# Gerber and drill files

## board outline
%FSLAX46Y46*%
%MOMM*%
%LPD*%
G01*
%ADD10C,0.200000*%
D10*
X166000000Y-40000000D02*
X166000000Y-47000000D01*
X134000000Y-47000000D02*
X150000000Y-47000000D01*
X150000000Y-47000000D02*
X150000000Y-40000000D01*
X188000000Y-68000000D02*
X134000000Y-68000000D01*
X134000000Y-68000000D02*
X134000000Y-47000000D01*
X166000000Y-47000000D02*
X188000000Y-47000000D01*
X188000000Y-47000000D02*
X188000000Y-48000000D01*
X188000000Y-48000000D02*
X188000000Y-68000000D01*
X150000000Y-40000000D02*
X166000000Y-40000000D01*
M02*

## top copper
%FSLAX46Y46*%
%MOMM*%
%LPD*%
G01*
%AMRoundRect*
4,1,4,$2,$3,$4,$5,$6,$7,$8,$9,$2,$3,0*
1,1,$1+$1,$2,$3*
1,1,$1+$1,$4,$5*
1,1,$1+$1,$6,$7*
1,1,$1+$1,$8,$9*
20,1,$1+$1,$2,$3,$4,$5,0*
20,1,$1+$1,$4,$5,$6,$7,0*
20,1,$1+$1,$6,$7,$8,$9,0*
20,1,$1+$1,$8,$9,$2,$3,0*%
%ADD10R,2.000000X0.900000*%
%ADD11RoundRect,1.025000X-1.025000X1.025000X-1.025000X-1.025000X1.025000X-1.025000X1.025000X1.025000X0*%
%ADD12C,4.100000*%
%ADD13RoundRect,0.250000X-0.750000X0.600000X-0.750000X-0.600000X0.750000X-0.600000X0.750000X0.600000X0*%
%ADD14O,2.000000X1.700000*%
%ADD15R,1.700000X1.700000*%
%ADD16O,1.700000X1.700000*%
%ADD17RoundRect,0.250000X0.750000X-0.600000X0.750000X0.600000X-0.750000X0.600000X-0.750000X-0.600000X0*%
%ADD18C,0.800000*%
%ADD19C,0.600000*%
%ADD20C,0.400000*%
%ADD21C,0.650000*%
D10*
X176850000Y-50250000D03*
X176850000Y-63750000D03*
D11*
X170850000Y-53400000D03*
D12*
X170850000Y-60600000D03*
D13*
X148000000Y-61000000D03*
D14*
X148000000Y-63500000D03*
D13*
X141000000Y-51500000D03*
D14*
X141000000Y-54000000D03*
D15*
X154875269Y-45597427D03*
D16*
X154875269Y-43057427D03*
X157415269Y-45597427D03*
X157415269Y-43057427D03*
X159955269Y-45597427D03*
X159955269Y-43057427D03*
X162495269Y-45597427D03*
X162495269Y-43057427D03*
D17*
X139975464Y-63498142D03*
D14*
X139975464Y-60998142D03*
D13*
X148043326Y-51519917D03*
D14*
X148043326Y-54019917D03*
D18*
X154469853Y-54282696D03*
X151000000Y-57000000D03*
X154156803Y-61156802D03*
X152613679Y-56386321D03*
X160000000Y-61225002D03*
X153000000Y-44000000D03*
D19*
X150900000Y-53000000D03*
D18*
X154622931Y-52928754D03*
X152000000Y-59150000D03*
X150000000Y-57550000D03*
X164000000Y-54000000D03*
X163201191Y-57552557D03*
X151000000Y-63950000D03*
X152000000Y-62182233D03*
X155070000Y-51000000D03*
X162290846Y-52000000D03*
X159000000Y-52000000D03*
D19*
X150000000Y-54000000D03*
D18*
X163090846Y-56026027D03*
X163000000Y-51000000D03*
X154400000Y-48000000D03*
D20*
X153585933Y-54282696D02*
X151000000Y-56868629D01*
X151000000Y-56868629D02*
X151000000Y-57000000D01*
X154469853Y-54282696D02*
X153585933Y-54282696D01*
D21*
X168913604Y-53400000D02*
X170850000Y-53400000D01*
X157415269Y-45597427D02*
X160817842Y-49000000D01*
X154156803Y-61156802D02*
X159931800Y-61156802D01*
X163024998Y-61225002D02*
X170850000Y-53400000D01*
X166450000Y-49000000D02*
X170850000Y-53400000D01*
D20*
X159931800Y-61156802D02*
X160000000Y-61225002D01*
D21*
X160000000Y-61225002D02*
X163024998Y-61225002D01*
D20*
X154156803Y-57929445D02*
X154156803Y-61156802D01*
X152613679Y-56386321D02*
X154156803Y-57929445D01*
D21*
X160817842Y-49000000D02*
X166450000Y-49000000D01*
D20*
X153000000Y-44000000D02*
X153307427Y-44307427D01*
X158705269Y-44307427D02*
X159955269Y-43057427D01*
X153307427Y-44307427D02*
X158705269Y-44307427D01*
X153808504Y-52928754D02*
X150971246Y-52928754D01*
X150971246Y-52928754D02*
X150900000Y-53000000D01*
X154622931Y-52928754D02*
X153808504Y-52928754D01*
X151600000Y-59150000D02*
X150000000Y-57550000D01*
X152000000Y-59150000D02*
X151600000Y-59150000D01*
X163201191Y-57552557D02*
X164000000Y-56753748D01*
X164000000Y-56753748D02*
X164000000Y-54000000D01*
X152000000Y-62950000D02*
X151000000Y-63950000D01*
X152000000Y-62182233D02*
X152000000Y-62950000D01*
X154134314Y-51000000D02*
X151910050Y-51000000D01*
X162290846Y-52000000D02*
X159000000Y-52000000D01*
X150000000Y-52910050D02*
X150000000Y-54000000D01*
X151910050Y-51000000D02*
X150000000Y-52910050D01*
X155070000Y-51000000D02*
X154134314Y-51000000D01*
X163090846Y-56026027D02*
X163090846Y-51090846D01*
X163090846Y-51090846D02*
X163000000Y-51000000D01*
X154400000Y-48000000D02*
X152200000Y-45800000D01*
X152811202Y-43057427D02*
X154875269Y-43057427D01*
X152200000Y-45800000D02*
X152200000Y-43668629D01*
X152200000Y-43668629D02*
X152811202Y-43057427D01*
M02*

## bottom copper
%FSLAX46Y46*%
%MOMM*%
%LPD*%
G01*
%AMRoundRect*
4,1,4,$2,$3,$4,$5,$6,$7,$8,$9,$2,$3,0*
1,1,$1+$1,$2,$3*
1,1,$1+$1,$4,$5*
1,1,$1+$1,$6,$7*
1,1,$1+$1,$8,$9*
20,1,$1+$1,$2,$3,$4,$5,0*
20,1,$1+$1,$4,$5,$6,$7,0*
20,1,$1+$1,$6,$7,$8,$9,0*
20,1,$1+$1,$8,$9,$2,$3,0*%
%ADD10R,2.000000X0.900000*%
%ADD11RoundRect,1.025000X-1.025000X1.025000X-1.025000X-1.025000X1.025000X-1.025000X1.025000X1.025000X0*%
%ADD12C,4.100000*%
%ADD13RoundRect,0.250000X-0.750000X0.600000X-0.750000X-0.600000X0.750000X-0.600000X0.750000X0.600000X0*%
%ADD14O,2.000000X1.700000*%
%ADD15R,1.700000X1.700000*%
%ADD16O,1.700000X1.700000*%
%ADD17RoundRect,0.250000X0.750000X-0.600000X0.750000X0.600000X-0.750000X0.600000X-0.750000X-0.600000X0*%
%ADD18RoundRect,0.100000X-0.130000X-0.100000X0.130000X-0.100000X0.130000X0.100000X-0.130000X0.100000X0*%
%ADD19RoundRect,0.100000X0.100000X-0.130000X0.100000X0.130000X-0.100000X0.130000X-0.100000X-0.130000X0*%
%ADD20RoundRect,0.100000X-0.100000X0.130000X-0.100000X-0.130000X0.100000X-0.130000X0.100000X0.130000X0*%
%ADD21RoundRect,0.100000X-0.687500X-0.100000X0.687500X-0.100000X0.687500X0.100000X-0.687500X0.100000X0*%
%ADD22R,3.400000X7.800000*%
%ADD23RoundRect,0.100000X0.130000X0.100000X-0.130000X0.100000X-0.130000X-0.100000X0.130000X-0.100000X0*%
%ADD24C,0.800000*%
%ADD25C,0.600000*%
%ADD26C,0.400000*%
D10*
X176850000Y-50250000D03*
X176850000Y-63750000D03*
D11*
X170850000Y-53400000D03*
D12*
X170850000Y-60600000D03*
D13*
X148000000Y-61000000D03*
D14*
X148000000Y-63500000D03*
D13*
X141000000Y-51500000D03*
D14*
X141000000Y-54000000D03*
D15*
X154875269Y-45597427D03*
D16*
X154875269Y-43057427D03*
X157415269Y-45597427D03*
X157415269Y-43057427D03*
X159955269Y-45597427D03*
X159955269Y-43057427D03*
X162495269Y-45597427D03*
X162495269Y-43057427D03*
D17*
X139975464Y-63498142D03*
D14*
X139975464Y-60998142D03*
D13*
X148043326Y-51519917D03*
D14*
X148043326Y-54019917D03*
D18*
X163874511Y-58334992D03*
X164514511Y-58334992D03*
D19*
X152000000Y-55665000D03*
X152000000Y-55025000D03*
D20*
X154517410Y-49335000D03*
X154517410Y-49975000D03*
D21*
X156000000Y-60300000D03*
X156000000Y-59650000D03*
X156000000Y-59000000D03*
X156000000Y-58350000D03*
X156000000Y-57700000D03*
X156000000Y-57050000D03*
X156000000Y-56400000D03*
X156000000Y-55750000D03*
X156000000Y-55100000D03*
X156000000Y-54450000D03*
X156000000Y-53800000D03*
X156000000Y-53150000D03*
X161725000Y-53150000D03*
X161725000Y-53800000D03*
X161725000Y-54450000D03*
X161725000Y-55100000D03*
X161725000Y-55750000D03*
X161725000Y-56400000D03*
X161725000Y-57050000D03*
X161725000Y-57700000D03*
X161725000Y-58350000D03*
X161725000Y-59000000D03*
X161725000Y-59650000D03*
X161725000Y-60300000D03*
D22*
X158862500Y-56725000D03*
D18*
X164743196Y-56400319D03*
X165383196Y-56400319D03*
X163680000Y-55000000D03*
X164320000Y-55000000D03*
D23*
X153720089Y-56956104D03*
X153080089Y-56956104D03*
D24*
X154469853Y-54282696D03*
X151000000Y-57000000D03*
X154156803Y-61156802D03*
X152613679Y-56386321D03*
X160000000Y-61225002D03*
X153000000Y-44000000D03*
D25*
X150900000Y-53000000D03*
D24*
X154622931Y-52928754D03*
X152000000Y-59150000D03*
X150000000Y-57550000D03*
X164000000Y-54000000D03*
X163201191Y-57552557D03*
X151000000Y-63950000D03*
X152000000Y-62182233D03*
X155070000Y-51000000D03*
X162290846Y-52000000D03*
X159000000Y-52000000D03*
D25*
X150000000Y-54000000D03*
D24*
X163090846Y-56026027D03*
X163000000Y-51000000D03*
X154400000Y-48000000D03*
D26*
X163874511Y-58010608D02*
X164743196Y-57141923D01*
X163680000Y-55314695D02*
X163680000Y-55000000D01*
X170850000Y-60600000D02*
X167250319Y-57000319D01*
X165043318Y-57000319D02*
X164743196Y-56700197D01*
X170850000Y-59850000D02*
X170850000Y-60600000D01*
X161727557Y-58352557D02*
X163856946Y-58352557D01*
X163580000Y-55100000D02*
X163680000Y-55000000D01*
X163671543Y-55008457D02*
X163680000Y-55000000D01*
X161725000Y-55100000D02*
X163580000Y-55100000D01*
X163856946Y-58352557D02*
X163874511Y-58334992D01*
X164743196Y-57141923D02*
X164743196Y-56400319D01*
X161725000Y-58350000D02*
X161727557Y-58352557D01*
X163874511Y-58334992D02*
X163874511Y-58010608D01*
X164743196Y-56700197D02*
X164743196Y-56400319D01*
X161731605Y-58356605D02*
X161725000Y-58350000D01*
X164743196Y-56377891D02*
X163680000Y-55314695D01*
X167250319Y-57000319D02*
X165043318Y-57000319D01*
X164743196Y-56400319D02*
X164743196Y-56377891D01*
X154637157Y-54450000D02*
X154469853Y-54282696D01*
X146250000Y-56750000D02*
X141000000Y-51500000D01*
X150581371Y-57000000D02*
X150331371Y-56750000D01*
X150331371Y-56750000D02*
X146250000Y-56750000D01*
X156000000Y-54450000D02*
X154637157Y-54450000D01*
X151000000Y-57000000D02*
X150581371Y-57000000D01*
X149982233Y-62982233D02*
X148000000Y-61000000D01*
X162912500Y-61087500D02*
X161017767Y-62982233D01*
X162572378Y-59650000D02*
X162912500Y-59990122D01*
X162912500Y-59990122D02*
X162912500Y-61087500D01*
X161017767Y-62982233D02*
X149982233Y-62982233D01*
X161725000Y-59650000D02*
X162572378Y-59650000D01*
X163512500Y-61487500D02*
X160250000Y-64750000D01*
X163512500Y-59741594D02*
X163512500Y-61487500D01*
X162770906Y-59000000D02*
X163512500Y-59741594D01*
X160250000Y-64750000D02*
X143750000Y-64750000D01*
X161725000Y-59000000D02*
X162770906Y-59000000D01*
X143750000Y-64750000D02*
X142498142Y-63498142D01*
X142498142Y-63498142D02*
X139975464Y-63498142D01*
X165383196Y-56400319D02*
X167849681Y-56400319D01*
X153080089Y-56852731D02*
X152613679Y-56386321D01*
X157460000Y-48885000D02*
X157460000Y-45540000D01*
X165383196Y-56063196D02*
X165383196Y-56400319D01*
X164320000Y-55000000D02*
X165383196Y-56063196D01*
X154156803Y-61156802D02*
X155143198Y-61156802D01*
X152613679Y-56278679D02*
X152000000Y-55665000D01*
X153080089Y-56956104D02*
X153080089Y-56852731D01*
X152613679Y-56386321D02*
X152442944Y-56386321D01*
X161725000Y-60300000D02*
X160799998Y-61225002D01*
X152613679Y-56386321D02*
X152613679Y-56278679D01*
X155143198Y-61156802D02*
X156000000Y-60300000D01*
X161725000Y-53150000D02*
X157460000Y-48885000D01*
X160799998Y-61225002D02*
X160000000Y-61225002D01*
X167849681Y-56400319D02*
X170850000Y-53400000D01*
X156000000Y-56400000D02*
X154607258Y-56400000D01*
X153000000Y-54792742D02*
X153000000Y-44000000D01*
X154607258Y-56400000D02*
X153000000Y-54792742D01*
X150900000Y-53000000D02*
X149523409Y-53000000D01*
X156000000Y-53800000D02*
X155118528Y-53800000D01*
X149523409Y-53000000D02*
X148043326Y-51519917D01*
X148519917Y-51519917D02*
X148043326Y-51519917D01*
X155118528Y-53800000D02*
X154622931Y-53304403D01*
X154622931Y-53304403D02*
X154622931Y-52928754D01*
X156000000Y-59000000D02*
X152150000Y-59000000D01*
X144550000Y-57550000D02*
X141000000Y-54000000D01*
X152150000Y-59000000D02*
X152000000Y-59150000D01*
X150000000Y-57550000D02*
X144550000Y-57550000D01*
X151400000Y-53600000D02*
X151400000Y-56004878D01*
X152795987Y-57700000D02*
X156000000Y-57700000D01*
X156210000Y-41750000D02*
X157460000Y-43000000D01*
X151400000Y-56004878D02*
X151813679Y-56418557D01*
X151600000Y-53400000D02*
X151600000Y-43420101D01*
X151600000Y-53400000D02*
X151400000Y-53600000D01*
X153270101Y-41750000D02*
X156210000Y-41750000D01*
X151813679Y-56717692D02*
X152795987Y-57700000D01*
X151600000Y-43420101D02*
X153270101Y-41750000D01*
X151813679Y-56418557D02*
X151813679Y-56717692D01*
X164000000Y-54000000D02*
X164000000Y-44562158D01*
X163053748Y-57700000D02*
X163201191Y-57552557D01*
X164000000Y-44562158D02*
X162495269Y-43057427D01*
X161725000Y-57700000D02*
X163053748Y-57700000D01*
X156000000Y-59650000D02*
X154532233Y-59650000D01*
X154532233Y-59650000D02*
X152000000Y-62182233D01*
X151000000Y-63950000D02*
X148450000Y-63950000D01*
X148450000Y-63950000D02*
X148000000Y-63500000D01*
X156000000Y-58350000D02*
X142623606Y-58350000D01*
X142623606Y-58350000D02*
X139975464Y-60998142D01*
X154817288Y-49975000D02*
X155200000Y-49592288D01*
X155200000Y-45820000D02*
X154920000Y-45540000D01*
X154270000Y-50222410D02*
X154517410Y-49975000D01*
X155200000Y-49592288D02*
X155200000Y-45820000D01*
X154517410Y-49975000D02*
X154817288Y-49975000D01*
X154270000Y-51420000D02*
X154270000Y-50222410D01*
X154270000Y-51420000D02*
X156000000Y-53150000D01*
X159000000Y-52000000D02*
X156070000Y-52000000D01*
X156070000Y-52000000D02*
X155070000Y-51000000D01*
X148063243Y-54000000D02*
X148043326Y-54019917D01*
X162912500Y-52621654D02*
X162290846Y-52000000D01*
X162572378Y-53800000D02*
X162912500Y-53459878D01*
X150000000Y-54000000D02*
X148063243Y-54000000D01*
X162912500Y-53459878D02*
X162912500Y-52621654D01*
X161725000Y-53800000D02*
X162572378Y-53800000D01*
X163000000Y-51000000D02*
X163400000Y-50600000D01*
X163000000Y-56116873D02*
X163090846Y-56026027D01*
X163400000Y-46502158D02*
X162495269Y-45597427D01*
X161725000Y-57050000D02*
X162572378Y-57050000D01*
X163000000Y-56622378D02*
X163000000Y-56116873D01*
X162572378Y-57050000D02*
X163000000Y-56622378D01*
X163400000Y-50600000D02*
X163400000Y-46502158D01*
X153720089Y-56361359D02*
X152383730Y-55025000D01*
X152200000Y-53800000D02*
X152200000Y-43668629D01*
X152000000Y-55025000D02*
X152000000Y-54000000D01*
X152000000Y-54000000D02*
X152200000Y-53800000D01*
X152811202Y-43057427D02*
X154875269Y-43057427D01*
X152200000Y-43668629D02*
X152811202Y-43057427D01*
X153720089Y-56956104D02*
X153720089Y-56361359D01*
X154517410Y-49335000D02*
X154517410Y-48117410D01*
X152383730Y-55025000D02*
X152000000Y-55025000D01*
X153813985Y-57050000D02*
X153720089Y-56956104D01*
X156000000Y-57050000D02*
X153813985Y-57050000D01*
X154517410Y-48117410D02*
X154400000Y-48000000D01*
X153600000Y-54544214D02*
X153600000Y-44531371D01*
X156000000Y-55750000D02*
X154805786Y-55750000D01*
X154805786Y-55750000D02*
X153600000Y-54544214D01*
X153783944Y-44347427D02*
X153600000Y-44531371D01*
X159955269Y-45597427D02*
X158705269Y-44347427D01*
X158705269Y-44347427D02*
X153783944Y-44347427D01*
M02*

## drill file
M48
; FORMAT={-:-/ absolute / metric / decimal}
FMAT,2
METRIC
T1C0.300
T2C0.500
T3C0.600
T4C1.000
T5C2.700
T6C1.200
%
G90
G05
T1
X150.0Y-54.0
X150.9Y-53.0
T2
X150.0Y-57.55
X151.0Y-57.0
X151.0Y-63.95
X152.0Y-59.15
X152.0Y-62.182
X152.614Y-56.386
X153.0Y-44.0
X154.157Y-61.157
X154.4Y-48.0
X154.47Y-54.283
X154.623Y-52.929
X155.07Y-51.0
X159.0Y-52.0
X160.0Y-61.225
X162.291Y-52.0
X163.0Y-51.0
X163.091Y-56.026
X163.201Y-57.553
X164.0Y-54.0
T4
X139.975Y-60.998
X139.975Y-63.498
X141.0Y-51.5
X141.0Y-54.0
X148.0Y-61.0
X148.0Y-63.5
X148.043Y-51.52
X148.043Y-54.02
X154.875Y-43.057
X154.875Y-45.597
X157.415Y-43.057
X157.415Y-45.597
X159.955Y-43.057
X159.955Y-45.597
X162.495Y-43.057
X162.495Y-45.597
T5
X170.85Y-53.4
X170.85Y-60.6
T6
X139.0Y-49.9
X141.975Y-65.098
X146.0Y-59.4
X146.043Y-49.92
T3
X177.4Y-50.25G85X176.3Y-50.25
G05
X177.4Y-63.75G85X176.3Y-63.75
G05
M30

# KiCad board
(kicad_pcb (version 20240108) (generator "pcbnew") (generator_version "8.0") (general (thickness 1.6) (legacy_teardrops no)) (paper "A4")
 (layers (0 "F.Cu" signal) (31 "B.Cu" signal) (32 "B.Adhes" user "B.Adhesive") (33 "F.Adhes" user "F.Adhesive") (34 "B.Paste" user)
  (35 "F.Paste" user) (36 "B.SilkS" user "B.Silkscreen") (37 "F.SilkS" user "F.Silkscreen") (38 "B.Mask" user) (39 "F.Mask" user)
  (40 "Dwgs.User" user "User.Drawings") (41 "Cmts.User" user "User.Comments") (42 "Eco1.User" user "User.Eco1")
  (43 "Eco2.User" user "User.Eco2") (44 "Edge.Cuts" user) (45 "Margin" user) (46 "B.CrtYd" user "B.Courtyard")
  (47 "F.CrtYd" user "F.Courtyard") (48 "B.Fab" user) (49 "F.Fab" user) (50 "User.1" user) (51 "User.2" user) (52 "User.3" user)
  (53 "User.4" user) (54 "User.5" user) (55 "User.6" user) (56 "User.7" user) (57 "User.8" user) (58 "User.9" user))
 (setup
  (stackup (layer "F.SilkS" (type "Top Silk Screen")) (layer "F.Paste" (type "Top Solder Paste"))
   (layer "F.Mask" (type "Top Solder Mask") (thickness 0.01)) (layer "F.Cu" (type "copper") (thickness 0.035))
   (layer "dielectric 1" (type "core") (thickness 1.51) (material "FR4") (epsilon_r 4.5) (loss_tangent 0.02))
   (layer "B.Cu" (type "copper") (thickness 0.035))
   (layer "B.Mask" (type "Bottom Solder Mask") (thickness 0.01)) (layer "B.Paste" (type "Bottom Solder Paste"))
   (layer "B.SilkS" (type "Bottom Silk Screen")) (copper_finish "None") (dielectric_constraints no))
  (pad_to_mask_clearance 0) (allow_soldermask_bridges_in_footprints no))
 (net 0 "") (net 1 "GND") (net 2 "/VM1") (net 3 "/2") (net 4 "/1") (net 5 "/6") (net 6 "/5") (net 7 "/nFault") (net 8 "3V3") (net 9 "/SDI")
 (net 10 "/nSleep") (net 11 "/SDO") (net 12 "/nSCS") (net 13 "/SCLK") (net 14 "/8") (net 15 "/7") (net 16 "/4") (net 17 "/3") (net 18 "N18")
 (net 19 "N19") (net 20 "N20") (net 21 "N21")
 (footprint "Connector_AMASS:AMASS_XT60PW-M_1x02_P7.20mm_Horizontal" (layer "F.Cu") (at 170.85 53.4 -90)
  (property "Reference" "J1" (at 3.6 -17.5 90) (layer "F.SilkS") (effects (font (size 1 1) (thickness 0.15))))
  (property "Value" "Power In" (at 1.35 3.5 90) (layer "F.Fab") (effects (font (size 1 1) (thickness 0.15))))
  (pad "" thru_hole rect (at -3.15 -6 270) (size 0.9 2) (drill oval 0.6 1.7) (layers "*.Cu" "*.Mask") (remove_unused_layers no))
  (pad "" thru_hole rect (at 10.35 -6 270) (size 0.9 2) (drill oval 0.6 1.7) (layers "*.Cu" "*.Mask") (remove_unused_layers no))
  (pad "1" thru_hole roundrect (at 0 0 270) (size 4.1 4.1) (drill 2.7) (layers "*.Cu" "*.Mask") (remove_unused_layers no)
   (roundrect_rratio 0.25) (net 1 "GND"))
  (pad "2" thru_hole circle (at 7.2 0 270) (size 4.1 4.1) (drill 2.7) (layers "*.Cu" "*.Mask") (remove_unused_layers no) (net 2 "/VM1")))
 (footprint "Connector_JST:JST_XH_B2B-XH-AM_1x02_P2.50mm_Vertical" (layer "F.Cu") (at 148 61 -90)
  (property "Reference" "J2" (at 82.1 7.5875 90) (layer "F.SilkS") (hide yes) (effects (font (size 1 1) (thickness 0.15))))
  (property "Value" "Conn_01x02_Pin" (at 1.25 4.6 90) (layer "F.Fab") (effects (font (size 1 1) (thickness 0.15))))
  (pad "" np_thru_hole circle (at -1.6 2 270) (size 1.2 1.2) (drill 1.2) (layers "*.Cu" "*.Mask"))
  (pad "1" thru_hole roundrect (at 0 0 270) (size 1.7 2) (drill 1) (layers "*.Cu" "*.Mask") (remove_unused_layers no)
   (roundrect_rratio 0.147059) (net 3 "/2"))
  (pad "2" thru_hole oval (at 2.5 0 270) (size 1.7 2) (drill 1) (layers "*.Cu" "*.Mask") (remove_unused_layers no) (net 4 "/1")))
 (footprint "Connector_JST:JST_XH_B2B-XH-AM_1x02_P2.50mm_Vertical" (layer "F.Cu") (at 141 51.5 -90)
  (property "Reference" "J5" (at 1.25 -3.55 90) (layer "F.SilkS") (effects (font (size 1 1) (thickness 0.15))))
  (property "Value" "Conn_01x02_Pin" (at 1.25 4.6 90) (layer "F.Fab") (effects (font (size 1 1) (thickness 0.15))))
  (pad "" np_thru_hole circle (at -1.6 2 270) (size 1.2 1.2) (drill 1.2) (layers "*.Cu" "*.Mask"))
  (pad "1" thru_hole roundrect (at 0 0 270) (size 1.7 2) (drill 1) (layers "*.Cu" "*.Mask") (remove_unused_layers no)
   (roundrect_rratio 0.147059) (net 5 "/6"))
  (pad "2" thru_hole oval (at 2.5 0 270) (size 1.7 2) (drill 1) (layers "*.Cu" "*.Mask") (remove_unused_layers no) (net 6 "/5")))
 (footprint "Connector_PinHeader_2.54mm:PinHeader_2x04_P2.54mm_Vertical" (layer "F.Cu") (at 154.875269 45.597427 90)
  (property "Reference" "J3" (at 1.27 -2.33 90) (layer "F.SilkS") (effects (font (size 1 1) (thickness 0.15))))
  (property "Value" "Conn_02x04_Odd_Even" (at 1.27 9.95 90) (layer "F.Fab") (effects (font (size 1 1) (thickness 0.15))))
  (pad "1" thru_hole rect (at 0 0 90) (size 1.7 1.7) (drill 1) (layers "*.Cu" "*.Mask") (remove_unused_layers no) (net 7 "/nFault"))
  (pad "2" thru_hole oval (at 2.54 0 90) (size 1.7 1.7) (drill 1) (layers "*.Cu" "*.Mask") (remove_unused_layers no) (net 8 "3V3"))
  (pad "3" thru_hole oval (at 0 2.54 90) (size 1.7 1.7) (drill 1) (layers "*.Cu" "*.Mask") (remove_unused_layers no) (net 1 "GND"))
  (pad "4" thru_hole oval (at 2.54 2.54 90) (size 1.7 1.7) (drill 1) (layers "*.Cu" "*.Mask") (remove_unused_layers no) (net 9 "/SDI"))
  (pad "5" thru_hole oval (at 0 5.08 90) (size 1.7 1.7) (drill 1) (layers "*.Cu" "*.Mask") (remove_unused_layers no) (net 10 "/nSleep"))
  (pad "6" thru_hole oval (at 2.54 5.08 90) (size 1.7 1.7) (drill 1) (layers "*.Cu" "*.Mask") (remove_unused_layers no) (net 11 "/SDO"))
  (pad "7" thru_hole oval (at 0 7.62 90) (size 1.7 1.7) (drill 1) (layers "*.Cu" "*.Mask") (remove_unused_layers no) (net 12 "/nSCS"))
  (pad "8" thru_hole oval (at 2.54 7.62 90) (size 1.7 1.7) (drill 1) (layers "*.Cu" "*.Mask") (remove_unused_layers no) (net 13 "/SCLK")))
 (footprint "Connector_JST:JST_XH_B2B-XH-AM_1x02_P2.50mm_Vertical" (layer "F.Cu") (at 139.975464 63.498142 90)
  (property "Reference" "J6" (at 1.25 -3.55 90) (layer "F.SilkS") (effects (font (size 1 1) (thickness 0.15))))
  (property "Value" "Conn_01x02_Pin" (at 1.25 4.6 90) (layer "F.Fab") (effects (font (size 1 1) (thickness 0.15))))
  (pad "" np_thru_hole circle (at -1.6 2 90) (size 1.2 1.2) (drill 1.2) (layers "*.Cu" "*.Mask"))
  (pad "1" thru_hole roundrect (at 0 0 90) (size 1.7 2) (drill 1) (layers "*.Cu" "*.Mask") (remove_unused_layers no)
   (roundrect_rratio 0.147059) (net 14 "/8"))
  (pad "2" thru_hole oval (at 2.5 0 90) (size 1.7 2) (drill 1) (layers "*.Cu" "*.Mask") (remove_unused_layers no) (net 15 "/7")))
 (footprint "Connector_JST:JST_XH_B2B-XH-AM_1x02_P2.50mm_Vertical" (layer "F.Cu") (at 148.043326 51.519917 -90)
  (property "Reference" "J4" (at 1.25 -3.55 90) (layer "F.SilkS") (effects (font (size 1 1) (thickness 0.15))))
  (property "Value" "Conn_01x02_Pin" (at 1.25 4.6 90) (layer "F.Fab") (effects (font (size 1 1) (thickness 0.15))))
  (pad "" np_thru_hole circle (at -1.6 2 270) (size 1.2 1.2) (drill 1.2) (layers "*.Cu" "*.Mask"))
  (pad "1" thru_hole roundrect (at 0 0 270) (size 1.7 2) (drill 1) (layers "*.Cu" "*.Mask") (remove_unused_layers no)
   (roundrect_rratio 0.147059) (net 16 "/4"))
  (pad "2" thru_hole oval (at 2.5 0 270) (size 1.7 2) (drill 1) (layers "*.Cu" "*.Mask") (remove_unused_layers no) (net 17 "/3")))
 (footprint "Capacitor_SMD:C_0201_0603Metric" (layer "B.Cu") (at 164.194511 58.334992)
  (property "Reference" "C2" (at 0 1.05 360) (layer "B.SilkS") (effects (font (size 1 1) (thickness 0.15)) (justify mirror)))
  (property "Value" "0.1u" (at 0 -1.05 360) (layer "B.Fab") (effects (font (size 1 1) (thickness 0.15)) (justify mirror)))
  (pad "" smd roundrect (at -0.345 0) (size 0.318 0.36) (layers "B.Paste") (roundrect_rratio 0.25))
  (pad "" smd roundrect (at 0.345 0) (size 0.318 0.36) (layers "B.Paste") (roundrect_rratio 0.25))
  (pad "1" smd roundrect (at -0.32 0) (size 0.46 0.4) (layers "B.Cu" "B.Mask") (roundrect_rratio 0.25) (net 2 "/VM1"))
  (pad "2" smd roundrect (at 0.32 0) (size 0.46 0.4) (layers "B.Cu" "B.Mask") (roundrect_rratio 0.25) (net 1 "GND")))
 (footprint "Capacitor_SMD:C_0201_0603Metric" (layer "B.Cu") (at 152 55.345 90)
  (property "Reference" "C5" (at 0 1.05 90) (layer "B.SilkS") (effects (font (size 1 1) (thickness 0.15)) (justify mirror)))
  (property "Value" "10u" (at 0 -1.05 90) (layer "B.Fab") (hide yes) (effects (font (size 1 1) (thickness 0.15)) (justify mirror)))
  (pad "" smd roundrect (at -0.345 0 90) (size 0.318 0.36) (layers "B.Paste") (roundrect_rratio 0.25))
  (pad "" smd roundrect (at 0.345 0 90) (size 0.318 0.36) (layers "B.Paste") (roundrect_rratio 0.25))
  (pad "1" smd roundrect (at -0.32 0 90) (size 0.46 0.4) (layers "B.Cu" "B.Mask") (roundrect_rratio 0.25) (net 1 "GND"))
  (pad "2" smd roundrect (at 0.32 0 90) (size 0.46 0.4) (layers "B.Cu" "B.Mask") (roundrect_rratio 0.25) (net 8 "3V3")))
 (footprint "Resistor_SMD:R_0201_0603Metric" (layer "B.Cu") (at 154.51741 49.655 -90)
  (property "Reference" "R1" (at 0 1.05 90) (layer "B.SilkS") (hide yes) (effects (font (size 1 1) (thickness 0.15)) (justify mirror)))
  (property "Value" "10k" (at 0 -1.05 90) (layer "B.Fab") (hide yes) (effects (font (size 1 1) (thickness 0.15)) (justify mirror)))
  (pad "" smd roundrect (at -0.345 0 270) (size 0.318 0.36) (layers "B.Paste") (roundrect_rratio 0.25))
  (pad "" smd roundrect (at 0.345 0 270) (size 0.318 0.36) (layers "B.Paste") (roundrect_rratio 0.25))
  (pad "1" smd roundrect (at -0.32 0 270) (size 0.46 0.4) (layers "B.Cu" "B.Mask") (roundrect_rratio 0.25) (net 8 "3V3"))
  (pad "2" smd roundrect (at 0.32 0 270) (size 0.46 0.4) (layers "B.Cu" "B.Mask") (roundrect_rratio 0.25) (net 7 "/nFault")))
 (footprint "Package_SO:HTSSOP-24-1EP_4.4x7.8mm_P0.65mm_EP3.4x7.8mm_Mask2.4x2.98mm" (layer "B.Cu") (at 158.8625 56.725)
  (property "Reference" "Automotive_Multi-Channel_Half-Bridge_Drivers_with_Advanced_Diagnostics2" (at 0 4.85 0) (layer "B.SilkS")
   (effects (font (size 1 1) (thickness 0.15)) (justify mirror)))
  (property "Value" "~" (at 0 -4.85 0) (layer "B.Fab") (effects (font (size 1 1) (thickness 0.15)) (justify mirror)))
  (pad "" smd roundrect (at 0 0) (size 1.93 2.4) (layers "B.Paste") (roundrect_rratio 0.129534))
  (pad "" smd rect (at 0 0) (size 2.4 2.98) (layers "B.Mask"))
  (pad "1" smd roundrect (at -2.8625 3.575) (size 1.575 0.4) (layers "B.Cu" "B.Paste" "B.Mask") (roundrect_rratio 0.25) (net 1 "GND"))
  (pad "2" smd roundrect (at -2.8625 2.925) (size 1.575 0.4) (layers "B.Cu" "B.Paste" "B.Mask") (roundrect_rratio 0.25) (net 4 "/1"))
  (pad "3" smd roundrect (at -2.8625 2.275) (size 1.575 0.4) (layers "B.Cu" "B.Paste" "B.Mask") (roundrect_rratio 0.25) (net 6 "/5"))
  (pad "4" smd roundrect (at -2.8625 1.625) (size 1.575 0.4) (layers "B.Cu" "B.Paste" "B.Mask") (roundrect_rratio 0.25) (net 15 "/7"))
  (pad "5" smd roundrect (at -2.8625 0.975) (size 1.575 0.4) (layers "B.Cu" "B.Paste" "B.Mask") (roundrect_rratio 0.25) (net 9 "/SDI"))
  (pad "6" smd roundrect (at -2.8625 0.325) (size 1.575 0.4) (layers "B.Cu" "B.Paste" "B.Mask") (roundrect_rratio 0.25) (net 8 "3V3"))
  (pad "7" smd roundrect (at -2.8625 -0.325) (size 1.575 0.4) (layers "B.Cu" "B.Paste" "B.Mask") (roundrect_rratio 0.25) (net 11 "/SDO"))
  (pad "8" smd roundrect (at -2.8625 -0.975) (size 1.575 0.4) (layers "B.Cu" "B.Paste" "B.Mask") (roundrect_rratio 0.25) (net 10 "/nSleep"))
  (pad "9" smd roundrect (at -2.8625 -1.625) (size 1.575 0.4) (layers "B.Cu" "B.Paste" "B.Mask") (roundrect_rratio 0.25) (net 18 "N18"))
  (pad "10" smd roundrect (at -2.8625 -2.275) (size 1.575 0.4) (layers "B.Cu" "B.Paste" "B.Mask") (roundrect_rratio 0.25) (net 5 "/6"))
  (pad "11" smd roundrect (at -2.8625 -2.925) (size 1.575 0.4) (layers "B.Cu" "B.Paste" "B.Mask") (roundrect_rratio 0.25) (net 16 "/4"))
  (pad "12" smd roundrect (at -2.8625 -3.575) (size 1.575 0.4) (layers "B.Cu" "B.Paste" "B.Mask") (roundrect_rratio 0.25) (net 7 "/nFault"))
  (pad "13" smd roundrect (at 2.8625 -3.575) (size 1.575 0.4) (layers "B.Cu" "B.Paste" "B.Mask") (roundrect_rratio 0.25) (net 1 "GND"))
  (pad "14" smd roundrect (at 2.8625 -2.925) (size 1.575 0.4) (layers "B.Cu" "B.Paste" "B.Mask") (roundrect_rratio 0.25) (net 17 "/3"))
  (pad "15" smd roundrect (at 2.8625 -2.275) (size 1.575 0.4) (layers "B.Cu" "B.Paste" "B.Mask") (roundrect_rratio 0.25) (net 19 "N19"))
  (pad "16" smd roundrect (at 2.8625 -1.625) (size 1.575 0.4) (layers "B.Cu" "B.Paste" "B.Mask") (roundrect_rratio 0.25) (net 2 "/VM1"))
  (pad "17" smd roundrect (at 2.8625 -0.975) (size 1.575 0.4) (layers "B.Cu" "B.Paste" "B.Mask") (roundrect_rratio 0.25) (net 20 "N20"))
  (pad "18" smd roundrect (at 2.8625 -0.325) (size 1.575 0.4) (layers "B.Cu" "B.Paste" "B.Mask") (roundrect_rratio 0.25) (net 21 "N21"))
  (pad "19" smd roundrect (at 2.8625 0.325) (size 1.575 0.4) (layers "B.Cu" "B.Paste" "B.Mask") (roundrect_rratio 0.25) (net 12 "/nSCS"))
  (pad "20" smd roundrect (at 2.8625 0.975) (size 1.575 0.4) (layers "B.Cu" "B.Paste" "B.Mask") (roundrect_rratio 0.25) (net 13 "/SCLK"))
  (pad "21" smd roundrect (at 2.8625 1.625) (size 1.575 0.4) (layers "B.Cu" "B.Paste" "B.Mask") (roundrect_rratio 0.25) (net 2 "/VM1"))
  (pad "22" smd roundrect (at 2.8625 2.275) (size 1.575 0.4) (layers "B.Cu" "B.Paste" "B.Mask") (roundrect_rratio 0.25) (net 14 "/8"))
  (pad "23" smd roundrect (at 2.8625 2.925) (size 1.575 0.4) (layers "B.Cu" "B.Paste" "B.Mask") (roundrect_rratio 0.25) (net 3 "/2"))
  (pad "24" smd roundrect (at 2.8625 3.575) (size 1.575 0.4) (layers "B.Cu" "B.Paste" "B.Mask") (roundrect_rratio 0.25) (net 1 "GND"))
  (pad "25" smd rect (at 0 0) (size 3.4 7.8) (layers "B.Cu") (zone_connect 2)))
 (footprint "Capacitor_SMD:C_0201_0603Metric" (layer "B.Cu") (at 165.063196 56.400319)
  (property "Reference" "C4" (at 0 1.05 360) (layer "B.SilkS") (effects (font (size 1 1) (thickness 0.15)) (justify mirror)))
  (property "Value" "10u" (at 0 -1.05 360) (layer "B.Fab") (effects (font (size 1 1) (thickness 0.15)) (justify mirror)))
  (pad "" smd roundrect (at -0.345 0) (size 0.318 0.36) (layers "B.Paste") (roundrect_rratio 0.25))
  (pad "" smd roundrect (at 0.345 0) (size 0.318 0.36) (layers "B.Paste") (roundrect_rratio 0.25))
  (pad "1" smd roundrect (at -0.32 0) (size 0.46 0.4) (layers "B.Cu" "B.Mask") (roundrect_rratio 0.25) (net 2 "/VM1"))
  (pad "2" smd roundrect (at 0.32 0) (size 0.46 0.4) (layers "B.Cu" "B.Mask") (roundrect_rratio 0.25) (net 1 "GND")))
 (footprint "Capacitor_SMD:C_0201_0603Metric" (layer "B.Cu") (at 164 55)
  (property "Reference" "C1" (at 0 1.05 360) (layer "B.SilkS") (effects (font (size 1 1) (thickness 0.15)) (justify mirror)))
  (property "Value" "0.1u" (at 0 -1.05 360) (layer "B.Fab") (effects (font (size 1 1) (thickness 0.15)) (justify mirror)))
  (pad "" smd roundrect (at -0.345 0) (size 0.318 0.36) (layers "B.Paste") (roundrect_rratio 0.25))
  (pad "" smd roundrect (at 0.345 0) (size 0.318 0.36) (layers "B.Paste") (roundrect_rratio 0.25))
  (pad "1" smd roundrect (at -0.32 0) (size 0.46 0.4) (layers "B.Cu" "B.Mask") (roundrect_rratio 0.25) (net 2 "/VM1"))
  (pad "2" smd roundrect (at 0.32 0) (size 0.46 0.4) (layers "B.Cu" "B.Mask") (roundrect_rratio 0.25) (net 1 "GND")))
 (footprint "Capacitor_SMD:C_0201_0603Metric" (layer "B.Cu") (at 153.400089 56.956104 180)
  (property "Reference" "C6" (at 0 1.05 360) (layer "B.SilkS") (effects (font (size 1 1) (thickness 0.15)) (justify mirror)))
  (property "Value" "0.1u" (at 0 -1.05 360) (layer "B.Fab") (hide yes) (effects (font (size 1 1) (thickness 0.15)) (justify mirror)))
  (pad "" smd roundrect (at -0.345 0 180) (size 0.318 0.36) (layers "B.Paste") (roundrect_rratio 0.25))
  (pad "" smd roundrect (at 0.345 0 180) (size 0.318 0.36) (layers "B.Paste") (roundrect_rratio 0.25))
  (pad "1" smd roundrect (at -0.32 0 180) (size 0.46 0.4) (layers "B.Cu" "B.Mask") (roundrect_rratio 0.25) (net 8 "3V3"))
  (pad "2" smd roundrect (at 0.32 0 180) (size 0.46 0.4) (layers "B.Cu" "B.Mask") (roundrect_rratio 0.25) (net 1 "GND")))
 (gr_line (start 166 40) (end 166 47) (stroke (width 0.2) (type default)) (layer "Edge.Cuts"))
 (gr_line (start 134 47) (end 150 47) (stroke (width 0.2) (type default)) (layer "Edge.Cuts"))
 (gr_line (start 150 47) (end 150 40) (stroke (width 0.2) (type default)) (layer "Edge.Cuts"))
 (gr_line (start 188 68) (end 134 68) (stroke (width 0.2) (type default)) (layer "Edge.Cuts"))
 (gr_line (start 134 68) (end 134 47) (stroke (width 0.2) (type default)) (layer "Edge.Cuts"))
 (gr_line (start 166 47) (end 188 47) (stroke (width 0.2) (type default)) (layer "Edge.Cuts"))
 (gr_line (start 188 47) (end 188 48) (stroke (width 0.2) (type default)) (layer "Edge.Cuts"))
 (gr_line (start 188 48) (end 188 68) (stroke (width 0.2) (type default)) (layer "Edge.Cuts"))
 (gr_line (start 150 40) (end 166 40) (stroke (width 0.2) (type default)) (layer "Edge.Cuts"))
 (segment (start 163.874511 58.010608) (end 164.743196 57.141923) (width 0.4) (layer "B.Cu") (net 2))
 (segment (start 163.68 55.314695) (end 163.68 55) (width 0.4) (layer "B.Cu") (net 2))
 (segment (start 170.85 60.6) (end 167.250319 57.000319) (width 0.4) (layer "B.Cu") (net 2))
 (segment (start 165.043318 57.000319) (end 164.743196 56.700197) (width 0.4) (layer "B.Cu") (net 2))
 (segment (start 170.85 59.85) (end 170.85 60.6) (width 0.4) (layer "B.Cu") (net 2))
 (segment (start 161.727557 58.352557) (end 163.856946 58.352557) (width 0.4) (layer "B.Cu") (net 2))
 (segment (start 163.58 55.1) (end 163.68 55) (width 0.4) (layer "B.Cu") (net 2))
 (segment (start 163.671543 55.008457) (end 163.68 55) (width 0.4) (layer "B.Cu") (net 2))
 (segment (start 161.725 55.1) (end 163.58 55.1) (width 0.4) (layer "B.Cu") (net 2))
 (segment (start 163.856946 58.352557) (end 163.874511 58.334992) (width 0.4) (layer "B.Cu") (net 2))
 (segment (start 164.743196 57.141923) (end 164.743196 56.400319) (width 0.4) (layer "B.Cu") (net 2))
 (segment (start 161.725 58.35) (end 161.727557 58.352557) (width 0.4) (layer "B.Cu") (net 2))
 (segment (start 163.874511 58.334992) (end 163.874511 58.010608) (width 0.4) (layer "B.Cu") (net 2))
 (segment (start 164.743196 56.700197) (end 164.743196 56.400319) (width 0.4) (layer "B.Cu") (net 2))
 (segment (start 161.731605 58.356605) (end 161.725 58.35) (width 0.4) (layer "B.Cu") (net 2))
 (segment (start 164.743196 56.377891) (end 163.68 55.314695) (width 0.4) (layer "B.Cu") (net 2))
 (segment (start 167.250319 57.000319) (end 165.043318 57.000319) (width 0.4) (layer "B.Cu") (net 2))
 (segment (start 164.743196 56.400319) (end 164.743196 56.377891) (width 0.4) (layer "B.Cu") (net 2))
 (segment (start 153.585933 54.282696) (end 151 56.868629) (width 0.4) (layer "F.Cu") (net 5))
 (segment (start 151 56.868629) (end 151 57) (width 0.4) (layer "F.Cu") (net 5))
 (segment (start 154.469853 54.282696) (end 153.585933 54.282696) (width 0.4) (layer "F.Cu") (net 5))
 (via (at 154.469853 54.282696) (size 0.8) (drill 0.5) (layers "F.Cu" "B.Cu") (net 5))
 (via (at 151 57) (size 0.8) (drill 0.5) (layers "F.Cu" "B.Cu") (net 5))
 (segment (start 154.637157 54.45) (end 154.469853 54.282696) (width 0.4) (layer "B.Cu") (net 5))
 (segment (start 146.25 56.75) (end 141 51.5) (width 0.4) (layer "B.Cu") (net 5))
 (segment (start 150.581371 57) (end 150.331371 56.75) (width 0.4) (layer "B.Cu") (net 5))
 (segment (start 150.331371 56.75) (end 146.25 56.75) (width 0.4) (layer "B.Cu") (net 5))
 (segment (start 156 54.45) (end 154.637157 54.45) (width 0.4) (layer "B.Cu") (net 5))
 (segment (start 151 57) (end 150.581371 57) (width 0.4) (layer "B.Cu") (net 5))
 (segment (start 149.982233 62.982233) (end 148 61) (width 0.4) (layer "B.Cu") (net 3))
 (segment (start 162.9125 61.0875) (end 161.017767 62.982233) (width 0.4) (layer "B.Cu") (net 3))
 (segment (start 162.572378 59.65) (end 162.9125 59.990122) (width 0.4) (layer "B.Cu") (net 3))
 (segment (start 162.9125 59.990122) (end 162.9125 61.0875) (width 0.4) (layer "B.Cu") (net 3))
 (segment (start 161.017767 62.982233) (end 149.982233 62.982233) (width 0.4) (layer "B.Cu") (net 3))
 (segment (start 161.725 59.65) (end 162.572378 59.65) (width 0.4) (layer "B.Cu") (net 3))
 (segment (start 163.5125 61.4875) (end 160.25 64.75) (width 0.4) (layer "B.Cu") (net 14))
 (segment (start 163.5125 59.741594) (end 163.5125 61.4875) (width 0.4) (layer "B.Cu") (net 14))
 (segment (start 162.770906 59) (end 163.5125 59.741594) (width 0.4) (layer "B.Cu") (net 14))
 (segment (start 160.25 64.75) (end 143.75 64.75) (width 0.4) (layer "B.Cu") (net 14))
 (segment (start 161.725 59) (end 162.770906 59) (width 0.4) (layer "B.Cu") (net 14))
 (segment (start 143.75 64.75) (end 142.498142 63.498142) (width 0.4) (layer "B.Cu") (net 14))
 (segment (start 142.498142 63.498142) (end 139.975464 63.498142) (width 0.4) (layer "B.Cu") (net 14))
 (segment (start 168.913604 53.4) (end 170.85 53.4) (width 0.65) (layer "F.Cu") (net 1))
 (segment (start 157.415269 45.597427) (end 160.817842 49) (width 0.65) (layer "F.Cu") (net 1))
 (segment (start 154.156803 61.156802) (end 159.9318 61.156802) (width 0.65) (layer "F.Cu") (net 1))
 (segment (start 163.024998 61.225002) (end 170.85 53.4) (width 0.65) (layer "F.Cu") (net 1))
 (segment (start 166.45 49) (end 170.85 53.4) (width 0.65) (layer "F.Cu") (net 1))
 (segment (start 159.9318 61.156802) (end 160 61.225002) (width 0.4) (layer "F.Cu") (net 1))
 (segment (start 160 61.225002) (end 163.024998 61.225002) (width 0.65) (layer "F.Cu") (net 1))
 (segment (start 154.156803 57.929445) (end 154.156803 61.156802) (width 0.4) (layer "F.Cu") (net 1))
 (segment (start 152.613679 56.386321) (end 154.156803 57.929445) (width 0.4) (layer "F.Cu") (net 1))
 (segment (start 160.817842 49) (end 166.45 49) (width 0.65) (layer "F.Cu") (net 1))
 (via (at 154.156803 61.156802) (size 0.8) (drill 0.5) (layers "F.Cu" "B.Cu") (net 1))
 (via (at 152.613679 56.386321) (size 0.8) (drill 0.5) (layers "F.Cu" "B.Cu") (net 1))
 (via (at 160 61.225002) (size 0.8) (drill 0.5) (layers "F.Cu" "B.Cu") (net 1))
 (segment (start 165.383196 56.400319) (end 167.849681 56.400319) (width 0.4) (layer "B.Cu") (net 1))
 (segment (start 153.080089 56.852731) (end 152.613679 56.386321) (width 0.4) (layer "B.Cu") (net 1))
 (segment (start 157.46 48.885) (end 157.46 45.54) (width 0.4) (layer "B.Cu") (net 1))
 (segment (start 165.383196 56.063196) (end 165.383196 56.400319) (width 0.4) (layer "B.Cu") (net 1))
 (segment (start 164.32 55) (end 165.383196 56.063196) (width 0.4) (layer "B.Cu") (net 1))
 (segment (start 154.156803 61.156802) (end 155.143198 61.156802) (width 0.4) (layer "B.Cu") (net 1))
 (segment (start 152.613679 56.278679) (end 152 55.665) (width 0.4) (layer "B.Cu") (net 1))
 (segment (start 153.080089 56.956104) (end 153.080089 56.852731) (width 0.4) (layer "B.Cu") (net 1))
 (segment (start 152.613679 56.386321) (end 152.442944 56.386321) (width 0.4) (layer "B.Cu") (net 1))
 (segment (start 161.725 60.3) (end 160.799998 61.225002) (width 0.4) (layer "B.Cu") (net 1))
 (segment (start 152.613679 56.386321) (end 152.613679 56.278679) (width 0.4) (layer "B.Cu") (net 1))
 (segment (start 155.143198 61.156802) (end 156 60.3) (width 0.4) (layer "B.Cu") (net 1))
 (segment (start 161.725 53.15) (end 157.46 48.885) (width 0.4) (layer "B.Cu") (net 1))
 (segment (start 160.799998 61.225002) (end 160 61.225002) (width 0.4) (layer "B.Cu") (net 1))
 (segment (start 167.849681 56.400319) (end 170.85 53.4) (width 0.4) (layer "B.Cu") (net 1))
 (segment (start 153 44) (end 153.307427 44.307427) (width 0.4) (layer "F.Cu") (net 11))
 (segment (start 158.705269 44.307427) (end 159.955269 43.057427) (width 0.4) (layer "F.Cu") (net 11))
 (segment (start 153.307427 44.307427) (end 158.705269 44.307427) (width 0.4) (layer "F.Cu") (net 11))
 (via (at 153 44) (size 0.8) (drill 0.5) (layers "F.Cu" "B.Cu") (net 11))
 (segment (start 156 56.4) (end 154.607258 56.4) (width 0.4) (layer "B.Cu") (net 11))
 (segment (start 153 54.792742) (end 153 44) (width 0.4) (layer "B.Cu") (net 11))
 (segment (start 154.607258 56.4) (end 153 54.792742) (width 0.4) (layer "B.Cu") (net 11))
 (segment (start 153.808504 52.928754) (end 150.971246 52.928754) (width 0.4) (layer "F.Cu") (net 16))
 (segment (start 150.971246 52.928754) (end 150.9 53) (width 0.4) (layer "F.Cu") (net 16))
 (segment (start 154.622931 52.928754) (end 153.808504 52.928754) (width 0.4) (layer "F.Cu") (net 16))
 (via (at 150.9 53) (size 0.6) (drill 0.3) (layers "F.Cu" "B.Cu") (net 16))
 (via (at 154.622931 52.928754) (size 0.8) (drill 0.5) (layers "F.Cu" "B.Cu") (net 16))
 (segment (start 150.9 53) (end 149.523409 53) (width 0.4) (layer "B.Cu") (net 16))
 (segment (start 156 53.8) (end 155.118528 53.8) (width 0.4) (layer "B.Cu") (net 16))
 (segment (start 149.523409 53) (end 148.043326 51.519917) (width 0.4) (layer "B.Cu") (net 16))
 (segment (start 148.519917 51.519917) (end 148.043326 51.519917) (width 0.4) (layer "B.Cu") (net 16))
 (segment (start 155.118528 53.8) (end 154.622931 53.304403) (width 0.4) (layer "B.Cu") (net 16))
 (segment (start 154.622931 53.304403) (end 154.622931 52.928754) (width 0.4) (layer "B.Cu") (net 16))
 (segment (start 151.6 59.15) (end 150 57.55) (width 0.4) (layer "F.Cu") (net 6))
 (segment (start 152 59.15) (end 151.6 59.15) (width 0.4) (layer "F.Cu") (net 6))
 (via (at 152 59.15) (size 0.8) (drill 0.5) (layers "F.Cu" "B.Cu") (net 6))
 (via (at 150 57.55) (size 0.8) (drill 0.5) (layers "F.Cu" "B.Cu") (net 6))
 (segment (start 156 59) (end 152.15 59) (width 0.4) (layer "B.Cu") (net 6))
 (segment (start 144.55 57.55) (end 141 54) (width 0.4) (layer "B.Cu") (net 6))
 (segment (start 152.15 59) (end 152 59.15) (width 0.4) (layer "B.Cu") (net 6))
 (segment (start 150 57.55) (end 144.55 57.55) (width 0.4) (layer "B.Cu") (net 6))
 (segment (start 151.4 53.6) (end 151.4 56.004878) (width 0.4) (layer "B.Cu") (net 9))
 (segment (start 152.795987 57.7) (end 156 57.7) (width 0.4) (layer "B.Cu") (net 9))
 (segment (start 156.21 41.75) (end 157.46 43) (width 0.4) (layer "B.Cu") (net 9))
 (segment (start 151.4 56.004878) (end 151.813679 56.418557) (width 0.4) (layer "B.Cu") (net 9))
 (segment (start 151.6 53.4) (end 151.6 43.420101) (width 0.4) (layer "B.Cu") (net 9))
 (segment (start 151.6 53.4) (end 151.4 53.6) (width 0.4) (layer "B.Cu") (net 9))
 (segment (start 153.270101 41.75) (end 156.21 41.75) (width 0.4) (layer "B.Cu") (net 9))
 (segment (start 151.813679 56.717692) (end 152.795987 57.7) (width 0.4) (layer "B.Cu") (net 9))
 (segment (start 151.6 43.420101) (end 153.270101 41.75) (width 0.4) (layer "B.Cu") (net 9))
 (segment (start 151.813679 56.418557) (end 151.813679 56.717692) (width 0.4) (layer "B.Cu") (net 9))
 (segment (start 163.201191 57.552557) (end 164 56.753748) (width 0.4) (layer "F.Cu") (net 13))
 (segment (start 164 56.753748) (end 164 54) (width 0.4) (layer "F.Cu") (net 13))
 (via (at 164 54) (size 0.8) (drill 0.5) (layers "F.Cu" "B.Cu") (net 13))
 (via (at 163.201191 57.552557) (size 0.8) (drill 0.5) (layers "F.Cu" "B.Cu") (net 13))
 (segment (start 164 54) (end 164 44.562158) (width 0.4) (layer "B.Cu") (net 13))
 (segment (start 163.053748 57.7) (end 163.201191 57.552557) (width 0.4) (layer "B.Cu") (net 13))
 (segment (start 164 44.562158) (end 162.495269 43.057427) (width 0.4) (layer "B.Cu") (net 13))
 (segment (start 161.725 57.7) (end 163.053748 57.7) (width 0.4) (layer "B.Cu") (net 13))
 (segment (start 152 62.95) (end 151 63.95) (width 0.4) (layer "F.Cu") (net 4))
 (segment (start 152 62.182233) (end 152 62.95) (width 0.4) (layer "F.Cu") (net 4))
 (via (at 151 63.95) (size 0.8) (drill 0.5) (layers "F.Cu" "B.Cu") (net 4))
 (via (at 152 62.182233) (size 0.8) (drill 0.5) (layers "F.Cu" "B.Cu") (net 4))
 (segment (start 156 59.65) (end 154.532233 59.65) (width 0.4) (layer "B.Cu") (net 4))
 (segment (start 154.532233 59.65) (end 152 62.182233) (width 0.4) (layer "B.Cu") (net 4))
 (segment (start 151 63.95) (end 148.45 63.95) (width 0.4) (layer "B.Cu") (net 4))
 (segment (start 148.45 63.95) (end 148 63.5) (width 0.4) (layer "B.Cu") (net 4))
 (segment (start 156 58.35) (end 142.623606 58.35) (width 0.4) (layer "B.Cu") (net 15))
 (segment (start 142.623606 58.35) (end 139.975464 60.998142) (width 0.4) (layer "B.Cu") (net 15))
 (segment (start 154.817288 49.975) (end 155.2 49.592288) (width 0.4) (layer "B.Cu") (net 7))
 (segment (start 155.2 45.82) (end 154.92 45.54) (width 0.4) (layer "B.Cu") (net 7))
 (segment (start 154.27 50.22241) (end 154.51741 49.975) (width 0.4) (layer "B.Cu") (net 7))
 (segment (start 155.2 49.592288) (end 155.2 45.82) (width 0.4) (layer "B.Cu") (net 7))
 (segment (start 154.51741 49.975) (end 154.817288 49.975) (width 0.4) (layer "B.Cu") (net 7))
 (segment (start 154.27 51.42) (end 154.27 50.22241) (width 0.4) (layer "B.Cu") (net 7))
 (segment (start 154.27 51.42) (end 156 53.15) (width 0.4) (layer "B.Cu") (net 7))
 (segment (start 154.134314 51) (end 151.91005 51) (width 0.4) (layer "F.Cu") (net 17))
 (segment (start 162.290846 52) (end 159 52) (width 0.4) (layer "F.Cu") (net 17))
 (segment (start 150 52.91005) (end 150 54) (width 0.4) (layer "F.Cu") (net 17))
 (segment (start 151.91005 51) (end 150 52.91005) (width 0.4) (layer "F.Cu") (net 17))
 (segment (start 155.07 51) (end 154.134314 51) (width 0.4) (layer "F.Cu") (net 17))
 (via (at 155.07 51) (size 0.8) (drill 0.5) (layers "F.Cu" "B.Cu") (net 17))
 (via (at 162.290846 52) (size 0.8) (drill 0.5) (layers "F.Cu" "B.Cu") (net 17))
 (via (at 159 52) (size 0.8) (drill 0.5) (layers "F.Cu" "B.Cu") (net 17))
 (via (at 150 54) (size 0.6) (drill 0.3) (layers "F.Cu" "B.Cu") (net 17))
 (segment (start 159 52) (end 156.07 52) (width 0.4) (layer "B.Cu") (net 17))
 (segment (start 156.07 52) (end 155.07 51) (width 0.4) (layer "B.Cu") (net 17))
 (segment (start 148.063243 54) (end 148.043326 54.019917) (width 0.4) (layer "B.Cu") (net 17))
 (segment (start 162.9125 52.621654) (end 162.290846 52) (width 0.4) (layer "B.Cu") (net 17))
 (segment (start 162.572378 53.8) (end 162.9125 53.459878) (width 0.4) (layer "B.Cu") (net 17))
 (segment (start 150 54) (end 148.063243 54) (width 0.4) (layer "B.Cu") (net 17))
 (segment (start 162.9125 53.459878) (end 162.9125 52.621654) (width 0.4) (layer "B.Cu") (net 17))
 (segment (start 161.725 53.8) (end 162.572378 53.8) (width 0.4) (layer "B.Cu") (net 17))
 (segment (start 163.090846 56.026027) (end 163.090846 51.090846) (width 0.4) (layer "F.Cu") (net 12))
 (segment (start 163.090846 51.090846) (end 163 51) (width 0.4) (layer "F.Cu") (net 12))
 (via (at 163.090846 56.026027) (size 0.8) (drill 0.5) (layers "F.Cu" "B.Cu") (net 12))
 (via (at 163 51) (size 0.8) (drill 0.5) (layers "F.Cu" "B.Cu") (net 12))
 (segment (start 163 51) (end 163.4 50.6) (width 0.4) (layer "B.Cu") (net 12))
 (segment (start 163 56.116873) (end 163.090846 56.026027) (width 0.4) (layer "B.Cu") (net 12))
 (segment (start 163.4 46.502158) (end 162.495269 45.597427) (width 0.4) (layer "B.Cu") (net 12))
 (segment (start 161.725 57.05) (end 162.572378 57.05) (width 0.4) (layer "B.Cu") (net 12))
 (segment (start 163 56.622378) (end 163 56.116873) (width 0.4) (layer "B.Cu") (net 12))
 (segment (start 162.572378 57.05) (end 163 56.622378) (width 0.4) (layer "B.Cu") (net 12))
 (segment (start 163.4 50.6) (end 163.4 46.502158) (width 0.4) (layer "B.Cu") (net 12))
 (segment (start 154.4 48) (end 152.2 45.8) (width 0.4) (layer "F.Cu") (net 8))
 (segment (start 152.811202 43.057427) (end 154.875269 43.057427) (width 0.4) (layer "F.Cu") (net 8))
 (segment (start 152.2 45.8) (end 152.2 43.668629) (width 0.4) (layer "F.Cu") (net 8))
 (segment (start 152.2 43.668629) (end 152.811202 43.057427) (width 0.4) (layer "F.Cu") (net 8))
 (via (at 154.4 48) (size 0.8) (drill 0.5) (layers "F.Cu" "B.Cu") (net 8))
 (segment (start 153.720089 56.361359) (end 152.38373 55.025) (width 0.4) (layer "B.Cu") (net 8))
 (segment (start 152.2 53.8) (end 152.2 43.668629) (width 0.4) (layer "B.Cu") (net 8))
 (segment (start 152 55.025) (end 152 54) (width 0.4) (layer "B.Cu") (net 8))
 (segment (start 152 54) (end 152.2 53.8) (width 0.4) (layer "B.Cu") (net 8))
 (segment (start 152.811202 43.057427) (end 154.875269 43.057427) (width 0.4) (layer "B.Cu") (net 8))
 (segment (start 152.2 43.668629) (end 152.811202 43.057427) (width 0.4) (layer "B.Cu") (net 8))
 (segment (start 153.720089 56.956104) (end 153.720089 56.361359) (width 0.4) (layer "B.Cu") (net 8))
 (segment (start 154.51741 49.335) (end 154.51741 48.11741) (width 0.4) (layer "B.Cu") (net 8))
 (segment (start 152.38373 55.025) (end 152 55.025) (width 0.4) (layer "B.Cu") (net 8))
 (segment (start 153.813985 57.05) (end 153.720089 56.956104) (width 0.4) (layer "B.Cu") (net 8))
 (segment (start 156 57.05) (end 153.813985 57.05) (width 0.4) (layer "B.Cu") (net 8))
 (segment (start 154.51741 48.11741) (end 154.4 48) (width 0.4) (layer "B.Cu") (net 8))
 (segment (start 153.6 54.544214) (end 153.6 44.531371) (width 0.4) (layer "B.Cu") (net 10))
 (segment (start 156 55.75) (end 154.805786 55.75) (width 0.4) (layer "B.Cu") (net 10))
 (segment (start 154.805786 55.75) (end 153.6 54.544214) (width 0.4) (layer "B.Cu") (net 10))
 (segment (start 153.783944 44.347427) (end 153.6 44.531371) (width 0.4) (layer "B.Cu") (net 10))
 (segment (start 159.955269 45.597427) (end 158.705269 44.347427) (width 0.4) (layer "B.Cu") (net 10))
 (segment (start 158.705269 44.347427) (end 153.783944 44.347427) (width 0.4) (layer "B.Cu") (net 10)))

